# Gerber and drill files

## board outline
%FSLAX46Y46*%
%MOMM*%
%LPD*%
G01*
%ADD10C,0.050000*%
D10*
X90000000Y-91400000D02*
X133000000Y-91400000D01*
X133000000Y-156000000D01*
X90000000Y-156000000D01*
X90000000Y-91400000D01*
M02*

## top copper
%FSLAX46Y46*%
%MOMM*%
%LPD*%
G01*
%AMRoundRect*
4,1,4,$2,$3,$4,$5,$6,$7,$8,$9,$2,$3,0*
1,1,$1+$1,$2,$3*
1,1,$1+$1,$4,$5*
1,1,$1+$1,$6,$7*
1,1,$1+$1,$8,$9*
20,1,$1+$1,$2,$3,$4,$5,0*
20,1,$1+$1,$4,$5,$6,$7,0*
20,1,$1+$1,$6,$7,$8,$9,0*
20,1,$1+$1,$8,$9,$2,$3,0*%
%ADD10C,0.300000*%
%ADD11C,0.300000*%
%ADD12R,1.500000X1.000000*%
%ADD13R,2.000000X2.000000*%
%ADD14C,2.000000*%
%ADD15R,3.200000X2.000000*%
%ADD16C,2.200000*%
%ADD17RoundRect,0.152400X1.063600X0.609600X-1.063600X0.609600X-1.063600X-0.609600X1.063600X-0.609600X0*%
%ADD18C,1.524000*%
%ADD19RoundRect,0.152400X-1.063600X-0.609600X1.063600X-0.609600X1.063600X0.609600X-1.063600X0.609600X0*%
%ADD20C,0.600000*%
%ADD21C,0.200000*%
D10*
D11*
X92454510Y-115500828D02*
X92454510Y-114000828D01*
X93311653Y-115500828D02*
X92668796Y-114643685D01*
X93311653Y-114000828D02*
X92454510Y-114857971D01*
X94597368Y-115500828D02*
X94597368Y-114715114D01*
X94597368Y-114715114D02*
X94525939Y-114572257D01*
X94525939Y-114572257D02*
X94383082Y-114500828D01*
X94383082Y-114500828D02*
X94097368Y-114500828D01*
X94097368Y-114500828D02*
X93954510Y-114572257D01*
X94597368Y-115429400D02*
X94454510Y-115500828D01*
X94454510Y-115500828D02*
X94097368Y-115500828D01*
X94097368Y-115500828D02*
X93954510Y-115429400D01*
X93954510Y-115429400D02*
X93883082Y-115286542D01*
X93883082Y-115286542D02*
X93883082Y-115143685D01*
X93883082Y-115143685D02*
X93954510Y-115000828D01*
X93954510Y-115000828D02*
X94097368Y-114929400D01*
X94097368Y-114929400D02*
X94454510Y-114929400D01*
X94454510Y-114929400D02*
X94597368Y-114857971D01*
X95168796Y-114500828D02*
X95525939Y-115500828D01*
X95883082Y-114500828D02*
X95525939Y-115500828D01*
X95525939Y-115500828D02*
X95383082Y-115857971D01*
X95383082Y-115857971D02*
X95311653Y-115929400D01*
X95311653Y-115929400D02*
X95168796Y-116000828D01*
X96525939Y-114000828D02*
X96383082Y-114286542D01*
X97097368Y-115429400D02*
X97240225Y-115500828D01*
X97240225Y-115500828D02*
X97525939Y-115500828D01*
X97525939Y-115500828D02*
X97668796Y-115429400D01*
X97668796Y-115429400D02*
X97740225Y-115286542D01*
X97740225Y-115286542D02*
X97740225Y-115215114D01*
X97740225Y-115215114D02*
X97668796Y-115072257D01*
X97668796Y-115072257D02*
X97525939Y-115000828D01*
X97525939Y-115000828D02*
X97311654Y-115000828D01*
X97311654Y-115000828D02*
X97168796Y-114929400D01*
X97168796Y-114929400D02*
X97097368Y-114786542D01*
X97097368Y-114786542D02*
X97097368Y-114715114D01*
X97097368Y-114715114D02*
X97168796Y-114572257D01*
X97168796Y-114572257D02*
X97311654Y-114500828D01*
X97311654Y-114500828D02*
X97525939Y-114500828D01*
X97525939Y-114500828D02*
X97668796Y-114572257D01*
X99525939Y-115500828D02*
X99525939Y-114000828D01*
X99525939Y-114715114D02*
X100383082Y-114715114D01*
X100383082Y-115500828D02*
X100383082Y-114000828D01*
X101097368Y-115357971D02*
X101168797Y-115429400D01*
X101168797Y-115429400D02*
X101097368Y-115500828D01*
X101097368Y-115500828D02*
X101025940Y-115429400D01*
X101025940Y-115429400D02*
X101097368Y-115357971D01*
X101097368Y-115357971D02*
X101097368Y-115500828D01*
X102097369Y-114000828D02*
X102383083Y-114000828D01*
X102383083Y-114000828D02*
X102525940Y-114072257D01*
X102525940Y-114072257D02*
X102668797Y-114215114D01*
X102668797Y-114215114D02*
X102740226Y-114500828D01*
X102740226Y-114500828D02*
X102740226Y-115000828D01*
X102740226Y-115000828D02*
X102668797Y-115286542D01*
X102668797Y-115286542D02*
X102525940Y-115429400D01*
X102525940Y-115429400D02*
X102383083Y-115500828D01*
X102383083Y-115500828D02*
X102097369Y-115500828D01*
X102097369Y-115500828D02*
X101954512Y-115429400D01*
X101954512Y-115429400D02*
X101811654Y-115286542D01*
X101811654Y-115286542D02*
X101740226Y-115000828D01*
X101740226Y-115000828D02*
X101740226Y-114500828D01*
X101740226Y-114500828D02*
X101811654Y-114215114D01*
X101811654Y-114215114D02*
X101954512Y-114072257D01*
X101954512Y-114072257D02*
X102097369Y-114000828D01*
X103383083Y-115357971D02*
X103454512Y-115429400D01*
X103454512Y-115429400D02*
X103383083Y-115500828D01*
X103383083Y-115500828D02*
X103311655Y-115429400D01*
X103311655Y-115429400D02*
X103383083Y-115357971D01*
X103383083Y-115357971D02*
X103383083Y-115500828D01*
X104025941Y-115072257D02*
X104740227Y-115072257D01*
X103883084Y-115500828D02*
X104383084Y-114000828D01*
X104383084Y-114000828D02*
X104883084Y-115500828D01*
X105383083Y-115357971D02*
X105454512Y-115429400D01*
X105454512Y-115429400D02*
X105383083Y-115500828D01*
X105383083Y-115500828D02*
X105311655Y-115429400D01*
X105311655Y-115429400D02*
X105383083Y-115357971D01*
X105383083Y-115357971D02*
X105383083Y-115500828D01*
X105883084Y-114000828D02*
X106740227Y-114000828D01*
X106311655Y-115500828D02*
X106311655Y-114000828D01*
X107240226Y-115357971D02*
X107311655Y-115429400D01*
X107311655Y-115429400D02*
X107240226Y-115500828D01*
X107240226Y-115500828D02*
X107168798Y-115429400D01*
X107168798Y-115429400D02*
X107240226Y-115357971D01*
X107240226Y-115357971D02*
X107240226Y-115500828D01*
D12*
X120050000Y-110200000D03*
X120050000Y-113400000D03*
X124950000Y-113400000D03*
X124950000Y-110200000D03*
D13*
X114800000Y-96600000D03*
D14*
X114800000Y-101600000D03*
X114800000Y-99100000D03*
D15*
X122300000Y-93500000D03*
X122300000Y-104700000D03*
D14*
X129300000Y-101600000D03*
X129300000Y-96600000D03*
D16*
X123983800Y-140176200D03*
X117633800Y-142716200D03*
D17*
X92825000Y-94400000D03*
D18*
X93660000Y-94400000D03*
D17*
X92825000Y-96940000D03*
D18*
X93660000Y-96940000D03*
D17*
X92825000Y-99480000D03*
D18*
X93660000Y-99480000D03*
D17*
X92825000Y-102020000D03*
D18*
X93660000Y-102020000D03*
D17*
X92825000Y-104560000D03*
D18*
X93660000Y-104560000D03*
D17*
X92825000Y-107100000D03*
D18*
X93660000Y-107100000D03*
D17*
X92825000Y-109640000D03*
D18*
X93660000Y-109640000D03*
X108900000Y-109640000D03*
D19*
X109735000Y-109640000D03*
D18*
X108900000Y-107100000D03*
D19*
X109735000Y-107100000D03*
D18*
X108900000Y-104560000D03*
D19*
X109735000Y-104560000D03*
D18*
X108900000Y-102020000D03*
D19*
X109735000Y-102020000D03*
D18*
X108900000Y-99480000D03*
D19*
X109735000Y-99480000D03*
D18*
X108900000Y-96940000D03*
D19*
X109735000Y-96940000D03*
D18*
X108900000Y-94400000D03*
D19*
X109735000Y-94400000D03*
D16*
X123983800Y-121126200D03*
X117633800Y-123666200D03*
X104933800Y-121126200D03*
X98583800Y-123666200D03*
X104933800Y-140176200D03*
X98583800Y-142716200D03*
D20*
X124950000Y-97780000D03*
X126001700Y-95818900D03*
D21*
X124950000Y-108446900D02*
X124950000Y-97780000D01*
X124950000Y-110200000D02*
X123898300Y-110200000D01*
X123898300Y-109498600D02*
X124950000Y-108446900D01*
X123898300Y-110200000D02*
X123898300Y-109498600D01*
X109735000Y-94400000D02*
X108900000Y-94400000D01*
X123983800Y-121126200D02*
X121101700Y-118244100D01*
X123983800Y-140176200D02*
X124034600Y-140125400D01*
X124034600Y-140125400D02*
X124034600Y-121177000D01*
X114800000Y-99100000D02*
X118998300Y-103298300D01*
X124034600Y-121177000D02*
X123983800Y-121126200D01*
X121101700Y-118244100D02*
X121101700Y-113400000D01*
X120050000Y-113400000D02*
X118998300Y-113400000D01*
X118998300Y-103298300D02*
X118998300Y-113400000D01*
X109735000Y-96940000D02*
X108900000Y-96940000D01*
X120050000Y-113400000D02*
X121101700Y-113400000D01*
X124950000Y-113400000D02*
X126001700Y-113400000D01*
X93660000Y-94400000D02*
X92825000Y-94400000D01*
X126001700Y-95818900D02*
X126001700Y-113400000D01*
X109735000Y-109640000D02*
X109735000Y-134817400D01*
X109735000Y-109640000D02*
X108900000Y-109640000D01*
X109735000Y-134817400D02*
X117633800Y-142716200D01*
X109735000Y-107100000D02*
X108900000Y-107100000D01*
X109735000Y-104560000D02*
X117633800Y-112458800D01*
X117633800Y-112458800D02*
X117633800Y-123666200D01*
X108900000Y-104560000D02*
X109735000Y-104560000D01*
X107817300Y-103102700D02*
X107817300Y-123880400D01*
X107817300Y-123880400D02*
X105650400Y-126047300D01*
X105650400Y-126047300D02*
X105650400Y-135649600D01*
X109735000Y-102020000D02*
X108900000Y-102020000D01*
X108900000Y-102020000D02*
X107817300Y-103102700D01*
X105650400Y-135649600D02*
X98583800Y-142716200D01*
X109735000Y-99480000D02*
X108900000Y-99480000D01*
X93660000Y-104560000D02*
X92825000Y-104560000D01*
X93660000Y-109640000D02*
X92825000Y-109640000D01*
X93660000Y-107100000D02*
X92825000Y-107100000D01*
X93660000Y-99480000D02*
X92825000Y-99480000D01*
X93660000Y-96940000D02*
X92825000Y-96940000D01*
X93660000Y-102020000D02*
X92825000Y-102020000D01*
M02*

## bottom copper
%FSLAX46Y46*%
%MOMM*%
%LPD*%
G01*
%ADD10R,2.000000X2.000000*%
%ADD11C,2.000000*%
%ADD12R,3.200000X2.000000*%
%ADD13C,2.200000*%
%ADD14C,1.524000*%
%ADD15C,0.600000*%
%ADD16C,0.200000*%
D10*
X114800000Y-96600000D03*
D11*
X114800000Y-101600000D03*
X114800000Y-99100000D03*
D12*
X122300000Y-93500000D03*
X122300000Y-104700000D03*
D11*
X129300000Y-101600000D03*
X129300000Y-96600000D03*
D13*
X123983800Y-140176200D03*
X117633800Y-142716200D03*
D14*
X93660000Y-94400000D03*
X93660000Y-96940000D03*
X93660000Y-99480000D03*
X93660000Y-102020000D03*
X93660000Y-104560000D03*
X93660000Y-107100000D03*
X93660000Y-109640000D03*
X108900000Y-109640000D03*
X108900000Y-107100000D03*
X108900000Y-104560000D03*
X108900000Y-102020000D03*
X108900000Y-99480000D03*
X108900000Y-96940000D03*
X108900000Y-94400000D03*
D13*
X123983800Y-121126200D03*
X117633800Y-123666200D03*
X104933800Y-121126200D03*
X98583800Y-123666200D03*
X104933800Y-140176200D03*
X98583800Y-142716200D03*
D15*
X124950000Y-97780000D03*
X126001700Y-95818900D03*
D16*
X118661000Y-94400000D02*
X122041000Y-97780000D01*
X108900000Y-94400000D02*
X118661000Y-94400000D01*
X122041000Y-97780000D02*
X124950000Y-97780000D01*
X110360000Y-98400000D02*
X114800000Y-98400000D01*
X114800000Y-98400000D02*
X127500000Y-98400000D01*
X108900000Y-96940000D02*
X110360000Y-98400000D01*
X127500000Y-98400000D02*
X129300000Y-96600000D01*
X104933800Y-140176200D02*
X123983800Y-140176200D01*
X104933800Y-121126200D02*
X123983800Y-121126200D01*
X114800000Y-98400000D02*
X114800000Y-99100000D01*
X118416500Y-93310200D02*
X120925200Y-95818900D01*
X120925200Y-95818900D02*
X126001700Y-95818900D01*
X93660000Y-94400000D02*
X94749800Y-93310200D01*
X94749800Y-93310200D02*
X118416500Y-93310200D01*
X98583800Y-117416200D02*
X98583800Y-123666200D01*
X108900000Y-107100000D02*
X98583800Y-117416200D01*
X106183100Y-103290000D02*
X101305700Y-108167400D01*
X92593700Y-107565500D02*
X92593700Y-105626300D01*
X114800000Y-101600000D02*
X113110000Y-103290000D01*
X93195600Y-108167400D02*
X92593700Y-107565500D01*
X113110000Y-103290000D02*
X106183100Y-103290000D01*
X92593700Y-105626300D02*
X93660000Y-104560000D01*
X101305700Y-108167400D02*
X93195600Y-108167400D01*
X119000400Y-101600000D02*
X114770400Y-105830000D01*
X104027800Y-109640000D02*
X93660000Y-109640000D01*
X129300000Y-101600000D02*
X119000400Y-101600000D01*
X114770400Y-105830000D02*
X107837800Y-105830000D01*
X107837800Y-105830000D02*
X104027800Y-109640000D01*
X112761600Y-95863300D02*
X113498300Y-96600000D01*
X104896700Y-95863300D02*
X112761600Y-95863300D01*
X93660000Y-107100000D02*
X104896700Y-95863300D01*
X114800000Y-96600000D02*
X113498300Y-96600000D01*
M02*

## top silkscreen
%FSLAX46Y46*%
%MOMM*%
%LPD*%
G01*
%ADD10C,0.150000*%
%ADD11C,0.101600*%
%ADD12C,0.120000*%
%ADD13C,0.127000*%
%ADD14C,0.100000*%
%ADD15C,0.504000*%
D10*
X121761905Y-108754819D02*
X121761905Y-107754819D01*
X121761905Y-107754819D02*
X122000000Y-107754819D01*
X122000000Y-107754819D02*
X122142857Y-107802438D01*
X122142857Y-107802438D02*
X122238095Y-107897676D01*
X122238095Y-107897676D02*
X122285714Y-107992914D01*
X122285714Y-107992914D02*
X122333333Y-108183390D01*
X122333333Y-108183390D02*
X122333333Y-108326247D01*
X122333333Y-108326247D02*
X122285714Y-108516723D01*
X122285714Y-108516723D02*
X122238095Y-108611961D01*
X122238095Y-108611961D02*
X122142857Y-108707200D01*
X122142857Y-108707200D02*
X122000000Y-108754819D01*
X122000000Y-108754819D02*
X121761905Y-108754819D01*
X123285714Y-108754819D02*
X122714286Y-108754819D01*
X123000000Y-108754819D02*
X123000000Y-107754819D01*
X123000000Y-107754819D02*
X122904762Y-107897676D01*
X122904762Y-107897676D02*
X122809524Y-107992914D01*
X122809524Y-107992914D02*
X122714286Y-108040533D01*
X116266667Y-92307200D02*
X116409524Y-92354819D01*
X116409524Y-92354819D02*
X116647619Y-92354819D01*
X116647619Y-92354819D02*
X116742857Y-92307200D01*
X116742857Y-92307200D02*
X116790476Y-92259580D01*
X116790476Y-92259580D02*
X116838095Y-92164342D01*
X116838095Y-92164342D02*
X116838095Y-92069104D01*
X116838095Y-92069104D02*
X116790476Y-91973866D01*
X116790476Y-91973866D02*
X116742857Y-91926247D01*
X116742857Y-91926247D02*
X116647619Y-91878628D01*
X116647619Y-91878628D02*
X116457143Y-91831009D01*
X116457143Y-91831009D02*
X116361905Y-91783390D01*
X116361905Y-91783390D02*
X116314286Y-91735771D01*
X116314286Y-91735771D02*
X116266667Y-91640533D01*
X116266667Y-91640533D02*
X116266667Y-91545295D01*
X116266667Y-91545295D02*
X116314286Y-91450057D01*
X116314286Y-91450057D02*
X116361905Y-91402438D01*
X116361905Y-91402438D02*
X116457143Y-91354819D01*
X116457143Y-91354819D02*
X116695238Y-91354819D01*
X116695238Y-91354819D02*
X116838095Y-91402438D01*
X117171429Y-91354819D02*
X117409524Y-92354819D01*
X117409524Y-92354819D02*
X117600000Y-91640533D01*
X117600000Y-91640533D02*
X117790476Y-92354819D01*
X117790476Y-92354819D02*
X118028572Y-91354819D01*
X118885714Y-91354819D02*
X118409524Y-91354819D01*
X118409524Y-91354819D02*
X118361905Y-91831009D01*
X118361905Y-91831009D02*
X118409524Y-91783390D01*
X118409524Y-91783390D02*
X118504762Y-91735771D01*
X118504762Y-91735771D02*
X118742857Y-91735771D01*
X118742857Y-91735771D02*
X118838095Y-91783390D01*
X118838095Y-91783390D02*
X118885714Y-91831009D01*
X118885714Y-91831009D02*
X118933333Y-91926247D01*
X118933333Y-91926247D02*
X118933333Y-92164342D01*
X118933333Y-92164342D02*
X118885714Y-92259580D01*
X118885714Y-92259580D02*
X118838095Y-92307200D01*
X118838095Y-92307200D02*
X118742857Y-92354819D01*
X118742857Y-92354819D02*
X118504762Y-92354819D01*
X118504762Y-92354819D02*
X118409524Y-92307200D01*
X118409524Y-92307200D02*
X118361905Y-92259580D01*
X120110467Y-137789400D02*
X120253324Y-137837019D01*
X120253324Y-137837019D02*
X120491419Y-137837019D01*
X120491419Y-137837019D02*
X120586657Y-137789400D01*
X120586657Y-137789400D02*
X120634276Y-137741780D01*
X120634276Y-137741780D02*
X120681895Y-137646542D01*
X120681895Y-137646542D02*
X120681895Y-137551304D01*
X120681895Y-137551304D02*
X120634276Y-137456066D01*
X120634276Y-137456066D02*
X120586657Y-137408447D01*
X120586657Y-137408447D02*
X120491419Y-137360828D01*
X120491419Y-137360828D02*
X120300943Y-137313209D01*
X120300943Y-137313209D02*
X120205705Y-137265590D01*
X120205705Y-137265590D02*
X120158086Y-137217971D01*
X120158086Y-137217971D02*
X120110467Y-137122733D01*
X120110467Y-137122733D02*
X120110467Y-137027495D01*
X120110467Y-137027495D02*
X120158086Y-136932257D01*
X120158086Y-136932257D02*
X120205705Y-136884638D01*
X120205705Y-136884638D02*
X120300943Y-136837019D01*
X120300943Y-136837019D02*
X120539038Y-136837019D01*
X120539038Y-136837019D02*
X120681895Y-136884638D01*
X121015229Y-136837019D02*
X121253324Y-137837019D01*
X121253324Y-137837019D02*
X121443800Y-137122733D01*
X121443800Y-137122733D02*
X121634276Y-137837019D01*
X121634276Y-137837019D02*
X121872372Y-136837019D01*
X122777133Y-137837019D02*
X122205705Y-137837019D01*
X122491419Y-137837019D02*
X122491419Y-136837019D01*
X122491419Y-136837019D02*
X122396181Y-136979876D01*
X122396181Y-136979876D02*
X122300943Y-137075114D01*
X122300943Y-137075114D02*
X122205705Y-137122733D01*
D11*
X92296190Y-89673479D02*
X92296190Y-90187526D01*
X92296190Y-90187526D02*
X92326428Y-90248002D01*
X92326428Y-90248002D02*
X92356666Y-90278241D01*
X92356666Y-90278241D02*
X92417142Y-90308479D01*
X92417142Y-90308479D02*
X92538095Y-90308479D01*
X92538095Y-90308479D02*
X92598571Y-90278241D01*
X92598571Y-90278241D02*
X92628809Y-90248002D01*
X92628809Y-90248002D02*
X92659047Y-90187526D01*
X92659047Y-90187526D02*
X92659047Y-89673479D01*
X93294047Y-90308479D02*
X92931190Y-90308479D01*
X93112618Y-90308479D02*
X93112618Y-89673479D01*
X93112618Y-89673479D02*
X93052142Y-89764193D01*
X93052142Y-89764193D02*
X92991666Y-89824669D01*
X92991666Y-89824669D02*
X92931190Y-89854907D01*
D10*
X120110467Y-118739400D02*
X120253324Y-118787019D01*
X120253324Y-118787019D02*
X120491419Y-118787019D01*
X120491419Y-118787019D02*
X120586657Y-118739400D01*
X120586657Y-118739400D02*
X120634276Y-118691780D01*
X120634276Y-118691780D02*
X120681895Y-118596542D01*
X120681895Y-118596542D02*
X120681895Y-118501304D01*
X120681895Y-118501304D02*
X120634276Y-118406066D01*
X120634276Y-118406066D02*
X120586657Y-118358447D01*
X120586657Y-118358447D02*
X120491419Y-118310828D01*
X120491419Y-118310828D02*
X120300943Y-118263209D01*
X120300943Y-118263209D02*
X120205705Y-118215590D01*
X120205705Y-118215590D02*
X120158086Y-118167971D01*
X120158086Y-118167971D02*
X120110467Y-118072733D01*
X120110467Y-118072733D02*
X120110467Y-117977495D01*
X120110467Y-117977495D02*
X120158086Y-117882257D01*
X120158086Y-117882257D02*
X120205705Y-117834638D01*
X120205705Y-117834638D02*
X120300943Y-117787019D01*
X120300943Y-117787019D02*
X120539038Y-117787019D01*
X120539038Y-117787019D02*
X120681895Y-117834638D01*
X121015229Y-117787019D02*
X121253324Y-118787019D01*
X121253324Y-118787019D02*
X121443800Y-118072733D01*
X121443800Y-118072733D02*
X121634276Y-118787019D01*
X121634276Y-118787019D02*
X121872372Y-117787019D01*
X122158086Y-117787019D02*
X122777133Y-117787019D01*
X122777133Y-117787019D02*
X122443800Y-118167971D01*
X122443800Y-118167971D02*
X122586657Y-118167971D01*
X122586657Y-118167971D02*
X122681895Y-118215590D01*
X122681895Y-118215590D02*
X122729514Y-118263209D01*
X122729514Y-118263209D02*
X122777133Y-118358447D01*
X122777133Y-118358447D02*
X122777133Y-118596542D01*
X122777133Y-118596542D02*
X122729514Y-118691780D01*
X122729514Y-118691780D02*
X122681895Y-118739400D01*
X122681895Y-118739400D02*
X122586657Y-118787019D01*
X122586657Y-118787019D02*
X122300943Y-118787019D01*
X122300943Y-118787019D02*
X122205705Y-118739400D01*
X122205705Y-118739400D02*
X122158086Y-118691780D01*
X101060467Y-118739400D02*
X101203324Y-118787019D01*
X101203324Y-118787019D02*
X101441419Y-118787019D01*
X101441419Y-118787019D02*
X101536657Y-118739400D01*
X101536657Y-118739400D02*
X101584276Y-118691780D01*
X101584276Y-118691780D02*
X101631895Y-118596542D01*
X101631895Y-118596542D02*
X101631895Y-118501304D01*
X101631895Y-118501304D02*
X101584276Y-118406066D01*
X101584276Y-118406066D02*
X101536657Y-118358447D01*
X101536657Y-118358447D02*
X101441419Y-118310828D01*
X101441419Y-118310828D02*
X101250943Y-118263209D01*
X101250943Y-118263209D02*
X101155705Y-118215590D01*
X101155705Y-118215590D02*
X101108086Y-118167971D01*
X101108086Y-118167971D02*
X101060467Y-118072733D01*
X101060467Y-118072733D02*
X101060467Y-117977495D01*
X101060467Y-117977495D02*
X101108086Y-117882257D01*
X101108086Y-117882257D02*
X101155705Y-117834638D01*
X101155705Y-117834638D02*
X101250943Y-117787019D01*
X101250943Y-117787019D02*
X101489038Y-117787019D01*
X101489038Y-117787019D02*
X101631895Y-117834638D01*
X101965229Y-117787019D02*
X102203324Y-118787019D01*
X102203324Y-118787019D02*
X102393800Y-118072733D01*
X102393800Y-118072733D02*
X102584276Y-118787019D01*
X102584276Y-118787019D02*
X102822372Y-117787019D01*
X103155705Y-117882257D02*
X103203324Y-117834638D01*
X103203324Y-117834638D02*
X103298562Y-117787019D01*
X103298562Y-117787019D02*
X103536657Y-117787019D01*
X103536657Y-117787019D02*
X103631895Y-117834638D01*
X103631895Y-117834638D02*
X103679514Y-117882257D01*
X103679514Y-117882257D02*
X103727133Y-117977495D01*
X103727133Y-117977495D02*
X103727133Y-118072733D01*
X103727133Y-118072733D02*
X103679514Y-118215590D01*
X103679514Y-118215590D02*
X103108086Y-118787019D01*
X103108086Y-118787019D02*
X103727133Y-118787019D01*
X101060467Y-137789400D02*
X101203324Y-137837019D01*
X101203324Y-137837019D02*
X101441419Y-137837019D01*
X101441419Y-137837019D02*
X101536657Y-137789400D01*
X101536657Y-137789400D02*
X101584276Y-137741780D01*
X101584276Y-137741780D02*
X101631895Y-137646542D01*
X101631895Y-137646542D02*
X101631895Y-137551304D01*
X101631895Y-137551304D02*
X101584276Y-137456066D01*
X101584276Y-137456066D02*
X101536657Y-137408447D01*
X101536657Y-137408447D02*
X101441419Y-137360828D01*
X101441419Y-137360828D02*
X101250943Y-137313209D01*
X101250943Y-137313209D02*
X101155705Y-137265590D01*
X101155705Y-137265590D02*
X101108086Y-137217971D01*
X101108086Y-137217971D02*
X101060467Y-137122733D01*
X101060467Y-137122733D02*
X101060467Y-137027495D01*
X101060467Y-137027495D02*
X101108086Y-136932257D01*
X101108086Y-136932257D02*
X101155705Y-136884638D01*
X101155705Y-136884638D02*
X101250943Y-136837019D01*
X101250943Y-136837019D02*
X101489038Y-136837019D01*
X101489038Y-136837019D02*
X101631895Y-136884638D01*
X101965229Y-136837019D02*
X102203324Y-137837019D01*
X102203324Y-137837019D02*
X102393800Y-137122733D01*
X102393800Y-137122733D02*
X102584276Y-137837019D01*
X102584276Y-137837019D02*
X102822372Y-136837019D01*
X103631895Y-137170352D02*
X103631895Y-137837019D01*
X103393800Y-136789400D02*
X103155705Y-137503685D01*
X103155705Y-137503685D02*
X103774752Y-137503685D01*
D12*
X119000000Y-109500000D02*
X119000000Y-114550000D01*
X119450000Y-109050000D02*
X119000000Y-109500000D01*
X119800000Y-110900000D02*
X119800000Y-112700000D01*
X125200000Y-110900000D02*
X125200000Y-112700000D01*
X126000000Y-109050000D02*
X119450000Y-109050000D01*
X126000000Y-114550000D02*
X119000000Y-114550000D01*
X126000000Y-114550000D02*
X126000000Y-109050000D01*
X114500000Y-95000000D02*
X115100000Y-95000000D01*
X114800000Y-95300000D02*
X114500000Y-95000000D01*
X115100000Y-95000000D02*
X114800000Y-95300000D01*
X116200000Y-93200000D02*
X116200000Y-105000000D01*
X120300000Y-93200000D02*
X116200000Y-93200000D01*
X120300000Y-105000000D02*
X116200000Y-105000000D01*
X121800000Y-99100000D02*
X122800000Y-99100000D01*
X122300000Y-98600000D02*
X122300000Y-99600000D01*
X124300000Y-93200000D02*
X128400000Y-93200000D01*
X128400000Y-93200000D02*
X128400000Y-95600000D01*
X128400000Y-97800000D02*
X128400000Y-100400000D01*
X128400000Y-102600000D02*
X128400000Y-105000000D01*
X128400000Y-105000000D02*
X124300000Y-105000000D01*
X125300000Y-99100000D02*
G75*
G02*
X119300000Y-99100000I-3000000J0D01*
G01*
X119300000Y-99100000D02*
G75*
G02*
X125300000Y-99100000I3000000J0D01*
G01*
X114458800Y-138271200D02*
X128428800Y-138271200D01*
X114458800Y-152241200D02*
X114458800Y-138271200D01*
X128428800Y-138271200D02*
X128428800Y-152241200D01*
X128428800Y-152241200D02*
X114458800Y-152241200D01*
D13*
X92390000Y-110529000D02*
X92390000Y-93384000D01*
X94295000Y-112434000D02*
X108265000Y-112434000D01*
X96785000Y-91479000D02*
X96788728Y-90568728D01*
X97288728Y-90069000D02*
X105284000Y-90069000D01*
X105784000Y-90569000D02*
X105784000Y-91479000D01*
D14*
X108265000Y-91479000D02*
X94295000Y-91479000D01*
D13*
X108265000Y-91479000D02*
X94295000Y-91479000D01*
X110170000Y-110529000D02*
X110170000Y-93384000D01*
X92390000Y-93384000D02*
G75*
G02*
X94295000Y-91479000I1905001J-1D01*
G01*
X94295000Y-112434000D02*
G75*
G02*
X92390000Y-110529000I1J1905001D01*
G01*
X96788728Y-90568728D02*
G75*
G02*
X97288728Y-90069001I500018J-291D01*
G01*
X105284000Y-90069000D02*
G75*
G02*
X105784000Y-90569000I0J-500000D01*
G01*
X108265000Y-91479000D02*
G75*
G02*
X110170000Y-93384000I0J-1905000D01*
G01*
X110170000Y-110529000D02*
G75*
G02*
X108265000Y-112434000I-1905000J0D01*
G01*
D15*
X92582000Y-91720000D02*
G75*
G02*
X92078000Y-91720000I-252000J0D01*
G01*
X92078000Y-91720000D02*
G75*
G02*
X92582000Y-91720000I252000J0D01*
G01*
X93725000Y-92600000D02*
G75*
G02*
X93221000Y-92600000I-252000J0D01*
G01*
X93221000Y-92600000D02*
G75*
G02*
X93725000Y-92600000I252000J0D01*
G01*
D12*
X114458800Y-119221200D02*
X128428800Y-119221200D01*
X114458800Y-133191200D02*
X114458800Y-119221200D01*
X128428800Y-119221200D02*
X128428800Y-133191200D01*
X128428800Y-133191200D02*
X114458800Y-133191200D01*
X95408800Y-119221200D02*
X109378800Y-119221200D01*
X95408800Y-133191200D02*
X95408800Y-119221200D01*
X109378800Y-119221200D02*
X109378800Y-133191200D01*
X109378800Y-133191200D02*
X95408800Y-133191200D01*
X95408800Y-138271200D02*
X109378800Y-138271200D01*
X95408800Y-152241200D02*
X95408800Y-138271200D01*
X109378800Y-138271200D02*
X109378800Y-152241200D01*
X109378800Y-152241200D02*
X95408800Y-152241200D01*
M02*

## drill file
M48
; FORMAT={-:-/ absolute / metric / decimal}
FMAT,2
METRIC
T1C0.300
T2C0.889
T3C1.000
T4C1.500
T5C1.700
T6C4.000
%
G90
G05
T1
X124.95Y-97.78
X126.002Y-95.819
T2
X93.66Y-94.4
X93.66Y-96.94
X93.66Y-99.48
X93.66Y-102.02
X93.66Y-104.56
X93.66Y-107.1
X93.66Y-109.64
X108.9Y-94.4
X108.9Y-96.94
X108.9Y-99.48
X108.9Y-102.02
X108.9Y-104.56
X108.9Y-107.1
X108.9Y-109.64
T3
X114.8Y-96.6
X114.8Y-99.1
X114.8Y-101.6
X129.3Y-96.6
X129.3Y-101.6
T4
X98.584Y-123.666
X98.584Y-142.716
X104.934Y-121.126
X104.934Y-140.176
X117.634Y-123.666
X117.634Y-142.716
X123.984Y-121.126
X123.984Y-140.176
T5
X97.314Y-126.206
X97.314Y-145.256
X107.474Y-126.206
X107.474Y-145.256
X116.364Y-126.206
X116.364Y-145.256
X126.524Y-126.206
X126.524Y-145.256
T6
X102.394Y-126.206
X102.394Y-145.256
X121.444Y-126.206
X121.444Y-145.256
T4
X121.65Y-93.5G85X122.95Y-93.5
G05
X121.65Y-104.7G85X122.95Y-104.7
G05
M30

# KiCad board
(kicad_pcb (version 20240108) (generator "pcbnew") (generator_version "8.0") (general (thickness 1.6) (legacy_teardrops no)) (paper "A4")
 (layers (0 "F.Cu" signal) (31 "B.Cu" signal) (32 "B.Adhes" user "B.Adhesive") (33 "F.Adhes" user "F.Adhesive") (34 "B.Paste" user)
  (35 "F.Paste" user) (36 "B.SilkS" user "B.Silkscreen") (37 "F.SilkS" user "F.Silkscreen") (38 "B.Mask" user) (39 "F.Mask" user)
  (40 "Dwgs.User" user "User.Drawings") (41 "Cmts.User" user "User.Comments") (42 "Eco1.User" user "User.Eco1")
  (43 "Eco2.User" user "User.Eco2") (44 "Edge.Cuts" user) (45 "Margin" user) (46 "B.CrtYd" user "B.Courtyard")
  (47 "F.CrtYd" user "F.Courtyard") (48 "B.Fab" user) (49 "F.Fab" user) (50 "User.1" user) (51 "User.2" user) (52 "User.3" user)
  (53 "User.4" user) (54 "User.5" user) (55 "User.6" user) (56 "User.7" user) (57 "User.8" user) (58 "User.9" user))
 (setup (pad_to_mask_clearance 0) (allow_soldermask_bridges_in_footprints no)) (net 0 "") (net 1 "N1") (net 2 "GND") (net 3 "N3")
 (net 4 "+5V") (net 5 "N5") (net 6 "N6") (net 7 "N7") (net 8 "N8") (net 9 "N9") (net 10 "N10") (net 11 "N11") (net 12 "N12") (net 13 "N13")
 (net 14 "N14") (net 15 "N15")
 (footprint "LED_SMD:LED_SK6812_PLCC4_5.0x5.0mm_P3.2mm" (layer "F.Cu") (at 122.5 111.8)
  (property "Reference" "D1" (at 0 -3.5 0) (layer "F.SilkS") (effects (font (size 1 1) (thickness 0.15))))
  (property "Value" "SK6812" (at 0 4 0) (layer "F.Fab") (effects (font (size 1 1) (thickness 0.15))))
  (fp_line (start -3.5 -2.3) (end -3.5 2.75) (stroke (width 0.12) (type default)) (layer "F.SilkS"))
  (fp_line (start -3.05 -2.75) (end -3.5 -2.3) (stroke (width 0.12) (type default)) (layer "F.SilkS"))
  (fp_line (start -2.7 -0.9) (end -2.7 0.9) (stroke (width 0.12) (type default)) (layer "F.SilkS"))
  (fp_line (start 2.7 -0.9) (end 2.7 0.9) (stroke (width 0.12) (type default)) (layer "F.SilkS"))
  (fp_line (start 3.5 -2.75) (end -3.05 -2.75) (stroke (width 0.12) (type solid)) (layer "F.SilkS"))
  (fp_line (start 3.5 2.75) (end -3.5 2.75) (stroke (width 0.12) (type solid)) (layer "F.SilkS"))
  (fp_line (start 3.5 2.75) (end 3.5 -2.75) (stroke (width 0.12) (type default)) (layer "F.SilkS"))
  (pad "1" smd rect (at -2.45 -1.6 180) (size 1.5 1) (layers "F.Cu" "F.Paste" "F.Mask") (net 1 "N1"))
  (pad "2" smd rect (at -2.45 1.6 180) (size 1.5 1) (layers "F.Cu" "F.Paste" "F.Mask") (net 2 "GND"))
  (pad "3" smd rect (at 2.45 1.6 180) (size 1.5 1) (layers "F.Cu" "F.Paste" "F.Mask") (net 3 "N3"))
  (pad "4" smd rect (at 2.45 -1.6 180) (size 1.5 1) (layers "F.Cu" "F.Paste" "F.Mask") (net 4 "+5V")))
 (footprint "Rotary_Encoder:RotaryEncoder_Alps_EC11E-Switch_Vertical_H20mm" (layer "F.Cu") (at 114.8 96.6)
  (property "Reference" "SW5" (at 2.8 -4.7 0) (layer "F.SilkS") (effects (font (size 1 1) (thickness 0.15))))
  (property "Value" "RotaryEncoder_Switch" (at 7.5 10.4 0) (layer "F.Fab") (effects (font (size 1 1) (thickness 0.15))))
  (fp_line (start -0.3 -1.6) (end 0.3 -1.6) (stroke (width 0.12) (type solid)) (layer "F.SilkS"))
  (fp_line (start 0 -1.3) (end -0.3 -1.6) (stroke (width 0.12) (type solid)) (layer "F.SilkS"))
  (fp_line (start 0.3 -1.6) (end 0 -1.3) (stroke (width 0.12) (type solid)) (layer "F.SilkS"))
  (fp_line (start 1.4 -3.4) (end 1.4 8.4) (stroke (width 0.12) (type solid)) (layer "F.SilkS"))
  (fp_line (start 5.5 -3.4) (end 1.4 -3.4) (stroke (width 0.12) (type solid)) (layer "F.SilkS"))
  (fp_line (start 5.5 8.4) (end 1.4 8.4) (stroke (width 0.12) (type solid)) (layer "F.SilkS"))
  (fp_line (start 7 2.5) (end 8 2.5) (stroke (width 0.12) (type solid)) (layer "F.SilkS"))
  (fp_line (start 7.5 2) (end 7.5 3) (stroke (width 0.12) (type solid)) (layer "F.SilkS"))
  (fp_line (start 9.5 -3.4) (end 13.6 -3.4) (stroke (width 0.12) (type solid)) (layer "F.SilkS"))
  (fp_line (start 13.6 -3.4) (end 13.6 -1) (stroke (width 0.12) (type solid)) (layer "F.SilkS"))
  (fp_line (start 13.6 1.2) (end 13.6 3.8) (stroke (width 0.12) (type solid)) (layer "F.SilkS"))
  (fp_line (start 13.6 6) (end 13.6 8.4) (stroke (width 0.12) (type solid)) (layer "F.SilkS"))
  (fp_line (start 13.6 8.4) (end 9.5 8.4) (stroke (width 0.12) (type solid)) (layer "F.SilkS"))
  (fp_circle (center 7.5 2.5) (end 10.5 2.5) (stroke (width 0.12) (type solid)) (fill none) (layer "F.SilkS"))
  (pad "A" thru_hole rect (at 0 0) (size 2 2) (drill 1) (layers "*.Cu" "*.Mask") (remove_unused_layers no) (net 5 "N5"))
  (pad "B" thru_hole circle (at 0 5) (size 2 2) (drill 1) (layers "*.Cu" "*.Mask") (remove_unused_layers no) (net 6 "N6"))
  (pad "C" thru_hole circle (at 0 2.5) (size 2 2) (drill 1) (layers "*.Cu" "*.Mask") (remove_unused_layers no) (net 2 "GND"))
  (pad "MP" thru_hole rect (at 7.5 -3.1) (size 3.2 2) (drill oval 2.8 1.5) (layers "*.Cu" "*.Mask") (remove_unused_layers no))
  (pad "MP" thru_hole rect (at 7.5 8.1) (size 3.2 2) (drill oval 2.8 1.5) (layers "*.Cu" "*.Mask") (remove_unused_layers no))
  (pad "S1" thru_hole circle (at 14.5 5) (size 2 2) (drill 1) (layers "*.Cu" "*.Mask") (remove_unused_layers no) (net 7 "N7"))
  (pad "S2" thru_hole circle (at 14.5 0) (size 2 2) (drill 1) (layers "*.Cu" "*.Mask") (remove_unused_layers no) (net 2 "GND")))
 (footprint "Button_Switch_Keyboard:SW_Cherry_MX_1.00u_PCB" (layer "F.Cu") (at 123.9838 140.1762)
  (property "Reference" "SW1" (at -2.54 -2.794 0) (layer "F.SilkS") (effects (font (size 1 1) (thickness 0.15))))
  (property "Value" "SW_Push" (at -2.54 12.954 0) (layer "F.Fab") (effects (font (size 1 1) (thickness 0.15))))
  (fp_line (start -9.525 -1.905) (end 4.445 -1.905) (stroke (width 0.12) (type solid)) (layer "F.SilkS"))
  (fp_line (start -9.525 12.065) (end -9.525 -1.905) (stroke (width 0.12) (type solid)) (layer "F.SilkS"))
  (fp_line (start 4.445 -1.905) (end 4.445 12.065) (stroke (width 0.12) (type solid)) (layer "F.SilkS"))
  (fp_line (start 4.445 12.065) (end -9.525 12.065) (stroke (width 0.12) (type solid)) (layer "F.SilkS"))
  (pad "" np_thru_hole circle (at -7.62 5.08) (size 1.7 1.7) (drill 1.7) (layers "*.Cu" "*.Mask"))
  (pad "" np_thru_hole circle (at -2.54 5.08) (size 4 4) (drill 4) (layers "*.Cu" "*.Mask"))
  (pad "" np_thru_hole circle (at 2.54 5.08) (size 1.7 1.7) (drill 1.7) (layers "*.Cu" "*.Mask"))
  (pad "1" thru_hole circle (at 0 0) (size 2.2 2.2) (drill 1.5) (layers "*.Cu" "*.Mask") (remove_unused_layers no) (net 2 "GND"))
  (pad "2" thru_hole circle (at -6.35 2.54) (size 2.2 2.2) (drill 1.5) (layers "*.Cu" "*.Mask") (remove_unused_layers no) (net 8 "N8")))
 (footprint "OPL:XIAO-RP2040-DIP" (layer "F.Cu") (at 101.28 102.02)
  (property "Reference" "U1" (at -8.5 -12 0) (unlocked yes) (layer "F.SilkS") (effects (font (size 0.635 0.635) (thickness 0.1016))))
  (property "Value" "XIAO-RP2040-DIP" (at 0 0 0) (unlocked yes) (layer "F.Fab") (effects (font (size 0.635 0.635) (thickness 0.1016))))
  (fp_line (start -8.89 8.509) (end -8.89 -8.636) (stroke (width 0.127) (type solid)) (layer "F.SilkS"))
  (fp_line (start -6.985 10.414) (end 6.985 10.414) (stroke (width 0.127) (type solid)) (layer "F.SilkS"))
  (fp_line (start -4.495 -10.541) (end -4.491272 -11.451272) (stroke (width 0.127) (type solid)) (layer "F.SilkS"))
  (fp_line (start -3.991272 -11.951) (end 4.004 -11.951) (stroke (width 0.127) (type solid)) (layer "F.SilkS"))
  (fp_line (start 4.504 -11.451) (end 4.504 -10.541) (stroke (width 0.127) (type solid)) (layer "F.SilkS"))
  (fp_line (start 6.985 -10.541) (end -6.985 -10.541) (stroke (width 0.1) (type solid)) (layer "F.SilkS"))
  (fp_line (start 6.985 -10.541) (end -6.985 -10.541) (stroke (width 0.127) (type solid)) (layer "F.SilkS"))
  (fp_line (start 8.89 8.509) (end 8.89 -8.636) (stroke (width 0.127) (type solid)) (layer "F.SilkS"))
  (fp_arc (start -8.89 -8.636) (mid -8.332038 -9.983038) (end -6.985 -10.541) (stroke (width 0.127) (type solid)) (layer "F.SilkS"))
  (fp_arc (start -6.985 10.414) (mid -8.332038 9.856038) (end -8.89 8.509) (stroke (width 0.127) (type solid)) (layer "F.SilkS"))
  (fp_arc (start -4.491272 -11.451272) (mid -4.344724 -11.804644) (end -3.991272 -11.951) (stroke (width 0.127) (type default))
   (layer "F.SilkS"))
  (fp_arc (start 4.004 -11.951) (mid 4.357553 -11.804553) (end 4.504 -11.451) (stroke (width 0.127) (type default)) (layer "F.SilkS"))
  (fp_arc (start 6.985 -10.541) (mid 8.332038 -9.983038) (end 8.89 -8.636) (stroke (width 0.127) (type solid)) (layer "F.SilkS"))
  (fp_arc (start 8.89 8.509) (mid 8.332038 9.856038) (end 6.985 10.414) (stroke (width 0.127) (type solid)) (layer "F.SilkS"))
  (fp_circle (center -8.95 -10.3) (end -8.95 -10.554) (stroke (width 0.5) (type solid)) (fill solid) (layer "F.SilkS"))
  (fp_circle (center -7.807 -9.42) (end -7.807 -9.674) (stroke (width 0.5) (type solid)) (fill solid) (layer "F.SilkS"))
  (pad "1" smd roundrect (at -8.455 -7.62 180) (size 2.432 1.524) (layers "F.Cu" "F.Mask") (roundrect_rratio 0.1) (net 3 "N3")
   (thermal_bridge_angle 45))
  (pad "1" thru_hole circle (at -7.62 -7.62 180) (size 1.524 1.524) (drill 0.889) (layers "*.Cu" "*.Mask") (remove_unused_layers no)
   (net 3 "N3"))
  (pad "2" smd roundrect (at -8.455 -5.08 180) (size 2.432 1.524) (layers "F.Cu" "F.Mask") (roundrect_rratio 0.1) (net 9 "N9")
   (thermal_bridge_angle 45))
  (pad "2" thru_hole circle (at -7.62 -5.08 180) (size 1.524 1.524) (drill 0.889) (layers "*.Cu" "*.Mask") (remove_unused_layers no)
   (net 9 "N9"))
  (pad "3" smd roundrect (at -8.455 -2.54 180) (size 2.432 1.524) (layers "F.Cu" "F.Mask") (roundrect_rratio 0.1) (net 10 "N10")
   (thermal_bridge_angle 45))
  (pad "3" thru_hole circle (at -7.62 -2.54 180) (size 1.524 1.524) (drill 0.889) (layers "*.Cu" "*.Mask") (remove_unused_layers no)
   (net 10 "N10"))
  (pad "4" smd roundrect (at -8.455 0 180) (size 2.432 1.524) (layers "F.Cu" "F.Mask") (roundrect_rratio 0.1) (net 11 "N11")
   (thermal_bridge_angle 45))
  (pad "4" thru_hole circle (at -7.62 0 180) (size 1.524 1.524) (drill 0.889) (layers "*.Cu" "*.Mask") (remove_unused_layers no)
   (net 11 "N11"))
  (pad "5" smd roundrect (at -8.455 2.54 180) (size 2.432 1.524) (layers "F.Cu" "F.Mask") (roundrect_rratio 0.1) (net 6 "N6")
   (thermal_bridge_angle 45))
  (pad "5" thru_hole circle (at -7.62 2.54 180) (size 1.524 1.524) (drill 0.889) (layers "*.Cu" "*.Mask") (remove_unused_layers no)
   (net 6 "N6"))
  (pad "6" smd roundrect (at -8.455 5.08 180) (size 2.432 1.524) (layers "F.Cu" "F.Mask") (roundrect_rratio 0.1) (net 5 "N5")
   (thermal_bridge_angle 45))
  (pad "6" thru_hole circle (at -7.62 5.08 180) (size 1.524 1.524) (drill 0.889) (layers "*.Cu" "*.Mask") (remove_unused_layers no)
   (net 5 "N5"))
  (pad "7" smd roundrect (at -8.455 7.62 180) (size 2.432 1.524) (layers "F.Cu" "F.Mask") (roundrect_rratio 0.1) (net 7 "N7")
   (thermal_bridge_angle 45))
  (pad "7" thru_hole circle (at -7.62 7.62 180) (size 1.524 1.524) (drill 0.889) (layers "*.Cu" "*.Mask") (remove_unused_layers no)
   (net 7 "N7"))
  (pad "8" thru_hole circle (at 7.62 7.62) (size 1.524 1.524) (drill 0.889) (layers "*.Cu" "*.Mask") (remove_unused_layers no) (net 8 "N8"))
  (pad "8" smd roundrect (at 8.455 7.62) (size 2.432 1.524) (layers "F.Cu" "F.Mask") (roundrect_rratio 0.1) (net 8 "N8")
   (thermal_bridge_angle 45))
  (pad "9" thru_hole circle (at 7.62 5.08) (size 1.524 1.524) (drill 0.889) (layers "*.Cu" "*.Mask") (remove_unused_layers no)
   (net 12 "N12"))
  (pad "9" smd roundrect (at 8.455 5.08) (size 2.432 1.524) (layers "F.Cu" "F.Mask") (roundrect_rratio 0.1) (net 12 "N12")
   (thermal_bridge_angle 45))
  (pad "10" thru_hole circle (at 7.62 2.54) (size 1.524 1.524) (drill 0.889) (layers "*.Cu" "*.Mask") (remove_unused_layers no)
   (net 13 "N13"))
  (pad "10" smd roundrect (at 8.455 2.54) (size 2.432 1.524) (layers "F.Cu" "F.Mask") (roundrect_rratio 0.1) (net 13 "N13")
   (thermal_bridge_angle 45))
  (pad "11" thru_hole circle (at 7.62 0) (size 1.524 1.524) (drill 0.889) (layers "*.Cu" "*.Mask") (remove_unused_layers no) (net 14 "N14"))
  (pad "11" smd roundrect (at 8.455 0) (size 2.432 1.524) (layers "F.Cu" "F.Mask") (roundrect_rratio 0.1) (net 14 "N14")
   (thermal_bridge_angle 45))
  (pad "12" thru_hole circle (at 7.62 -2.54) (size 1.524 1.524) (drill 0.889) (layers "*.Cu" "*.Mask") (remove_unused_layers no)
   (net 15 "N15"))
  (pad "12" smd roundrect (at 8.455 -2.54) (size 2.432 1.524) (layers "F.Cu" "F.Mask") (roundrect_rratio 0.1) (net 15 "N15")
   (thermal_bridge_angle 45))
  (pad "13" thru_hole circle (at 7.62 -5.08) (size 1.524 1.524) (drill 0.889) (layers "*.Cu" "*.Mask") (remove_unused_layers no)
   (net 2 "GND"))
  (pad "13" smd roundrect (at 8.455 -5.08) (size 2.432 1.524) (layers "F.Cu" "F.Mask") (roundrect_rratio 0.1) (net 2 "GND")
   (thermal_bridge_angle 45))
  (pad "14" thru_hole circle (at 7.62 -7.62) (size 1.524 1.524) (drill 0.889) (layers "*.Cu" "*.Mask") (remove_unused_layers no)
   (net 4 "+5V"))
  (pad "14" smd roundrect (at 8.455 -7.62) (size 2.432 1.524) (layers "F.Cu" "F.Mask") (roundrect_rratio 0.1) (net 4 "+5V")
   (thermal_bridge_angle 45)))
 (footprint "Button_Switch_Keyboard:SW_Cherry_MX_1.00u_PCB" (layer "F.Cu") (at 123.9838 121.1262)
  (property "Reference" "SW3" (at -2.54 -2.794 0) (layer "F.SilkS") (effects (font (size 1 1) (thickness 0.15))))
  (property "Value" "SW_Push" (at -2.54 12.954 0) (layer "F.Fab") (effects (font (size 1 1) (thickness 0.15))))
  (fp_line (start -9.525 -1.905) (end 4.445 -1.905) (stroke (width 0.12) (type solid)) (layer "F.SilkS"))
  (fp_line (start -9.525 12.065) (end -9.525 -1.905) (stroke (width 0.12) (type solid)) (layer "F.SilkS"))
  (fp_line (start 4.445 -1.905) (end 4.445 12.065) (stroke (width 0.12) (type solid)) (layer "F.SilkS"))
  (fp_line (start 4.445 12.065) (end -9.525 12.065) (stroke (width 0.12) (type solid)) (layer "F.SilkS"))
  (pad "" np_thru_hole circle (at -7.62 5.08) (size 1.7 1.7) (drill 1.7) (layers "*.Cu" "*.Mask"))
  (pad "" np_thru_hole circle (at -2.54 5.08) (size 4 4) (drill 4) (layers "*.Cu" "*.Mask"))
  (pad "" np_thru_hole circle (at 2.54 5.08) (size 1.7 1.7) (drill 1.7) (layers "*.Cu" "*.Mask"))
  (pad "1" thru_hole circle (at 0 0) (size 2.2 2.2) (drill 1.5) (layers "*.Cu" "*.Mask") (remove_unused_layers no) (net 2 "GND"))
  (pad "2" thru_hole circle (at -6.35 2.54) (size 2.2 2.2) (drill 1.5) (layers "*.Cu" "*.Mask") (remove_unused_layers no) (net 13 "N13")))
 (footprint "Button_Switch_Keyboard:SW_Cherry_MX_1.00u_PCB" (layer "F.Cu") (at 104.9338 121.1262)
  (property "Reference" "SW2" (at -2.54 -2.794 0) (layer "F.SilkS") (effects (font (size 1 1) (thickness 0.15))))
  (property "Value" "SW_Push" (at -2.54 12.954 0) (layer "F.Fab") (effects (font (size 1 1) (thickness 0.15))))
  (fp_line (start -9.525 -1.905) (end 4.445 -1.905) (stroke (width 0.12) (type solid)) (layer "F.SilkS"))
  (fp_line (start -9.525 12.065) (end -9.525 -1.905) (stroke (width 0.12) (type solid)) (layer "F.SilkS"))
  (fp_line (start 4.445 -1.905) (end 4.445 12.065) (stroke (width 0.12) (type solid)) (layer "F.SilkS"))
  (fp_line (start 4.445 12.065) (end -9.525 12.065) (stroke (width 0.12) (type solid)) (layer "F.SilkS"))
  (pad "" np_thru_hole circle (at -7.62 5.08) (size 1.7 1.7) (drill 1.7) (layers "*.Cu" "*.Mask"))
  (pad "" np_thru_hole circle (at -2.54 5.08) (size 4 4) (drill 4) (layers "*.Cu" "*.Mask"))
  (pad "" np_thru_hole circle (at 2.54 5.08) (size 1.7 1.7) (drill 1.7) (layers "*.Cu" "*.Mask"))
  (pad "1" thru_hole circle (at 0 0) (size 2.2 2.2) (drill 1.5) (layers "*.Cu" "*.Mask") (remove_unused_layers no) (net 2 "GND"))
  (pad "2" thru_hole circle (at -6.35 2.54) (size 2.2 2.2) (drill 1.5) (layers "*.Cu" "*.Mask") (remove_unused_layers no) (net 12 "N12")))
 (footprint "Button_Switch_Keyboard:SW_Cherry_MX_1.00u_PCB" (layer "F.Cu") (at 104.9338 140.1762)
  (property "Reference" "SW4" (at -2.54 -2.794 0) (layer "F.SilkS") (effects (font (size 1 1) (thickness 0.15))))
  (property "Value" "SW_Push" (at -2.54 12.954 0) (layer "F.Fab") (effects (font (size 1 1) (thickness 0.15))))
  (fp_line (start -9.525 -1.905) (end 4.445 -1.905) (stroke (width 0.12) (type solid)) (layer "F.SilkS"))
  (fp_line (start -9.525 12.065) (end -9.525 -1.905) (stroke (width 0.12) (type solid)) (layer "F.SilkS"))
  (fp_line (start 4.445 -1.905) (end 4.445 12.065) (stroke (width 0.12) (type solid)) (layer "F.SilkS"))
  (fp_line (start 4.445 12.065) (end -9.525 12.065) (stroke (width 0.12) (type solid)) (layer "F.SilkS"))
  (pad "" np_thru_hole circle (at -7.62 5.08) (size 1.7 1.7) (drill 1.7) (layers "*.Cu" "*.Mask"))
  (pad "" np_thru_hole circle (at -2.54 5.08) (size 4 4) (drill 4) (layers "*.Cu" "*.Mask"))
  (pad "" np_thru_hole circle (at 2.54 5.08) (size 1.7 1.7) (drill 1.7) (layers "*.Cu" "*.Mask"))
  (pad "1" thru_hole circle (at 0 0) (size 2.2 2.2) (drill 1.5) (layers "*.Cu" "*.Mask") (remove_unused_layers no) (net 2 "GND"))
  (pad "2" thru_hole circle (at -6.35 2.54) (size 2.2 2.2) (drill 1.5) (layers "*.Cu" "*.Mask") (remove_unused_layers no) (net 14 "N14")))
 (gr_rect (start 90 91.4) (end 133 156) (stroke (width 0.05) (type default)) (fill none) (layer "Edge.Cuts"))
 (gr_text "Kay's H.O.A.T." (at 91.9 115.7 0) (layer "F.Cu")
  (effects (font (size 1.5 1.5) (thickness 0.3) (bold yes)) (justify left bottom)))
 (segment (start 124.95 108.4469) (end 124.95 97.78) (width 0.2) (layer "F.Cu") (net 4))
 (segment (start 124.95 110.2) (end 123.8983 110.2) (width 0.2) (layer "F.Cu") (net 4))
 (segment (start 123.8983 109.4986) (end 124.95 108.4469) (width 0.2) (layer "F.Cu") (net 4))
 (segment (start 123.8983 110.2) (end 123.8983 109.4986) (width 0.2) (layer "F.Cu") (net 4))
 (segment (start 109.735 94.4) (end 108.9 94.4) (width 0.2) (layer "F.Cu") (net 4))
 (via (at 124.95 97.78) (size 0.6) (drill 0.3) (layers "F.Cu" "B.Cu") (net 4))
 (segment (start 118.661 94.4) (end 122.041 97.78) (width 0.2) (layer "B.Cu") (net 4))
 (segment (start 108.9 94.4) (end 118.661 94.4) (width 0.2) (layer "B.Cu") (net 4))
 (segment (start 122.041 97.78) (end 124.95 97.78) (width 0.2) (layer "B.Cu") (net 4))
 (segment (start 123.9838 121.1262) (end 121.1017 118.2441) (width 0.2) (layer "F.Cu") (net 2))
 (segment (start 123.9838 140.1762) (end 124.0346 140.1254) (width 0.2) (layer "F.Cu") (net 2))
 (segment (start 124.0346 140.1254) (end 124.0346 121.177) (width 0.2) (layer "F.Cu") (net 2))
 (segment (start 114.8 99.1) (end 118.9983 103.2983) (width 0.2) (layer "F.Cu") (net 2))
 (segment (start 124.0346 121.177) (end 123.9838 121.1262) (width 0.2) (layer "F.Cu") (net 2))
 (segment (start 121.1017 118.2441) (end 121.1017 113.4) (width 0.2) (layer "F.Cu") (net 2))
 (segment (start 120.05 113.4) (end 118.9983 113.4) (width 0.2) (layer "F.Cu") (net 2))
 (segment (start 118.9983 103.2983) (end 118.9983 113.4) (width 0.2) (layer "F.Cu") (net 2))
 (segment (start 109.735 96.94) (end 108.9 96.94) (width 0.2) (layer "F.Cu") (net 2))
 (segment (start 120.05 113.4) (end 121.1017 113.4) (width 0.2) (layer "F.Cu") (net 2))
 (segment (start 110.36 98.4) (end 114.8 98.4) (width 0.2) (layer "B.Cu") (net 2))
 (segment (start 114.8 98.4) (end 127.5 98.4) (width 0.2) (layer "B.Cu") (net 2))
 (segment (start 108.9 96.94) (end 110.36 98.4) (width 0.2) (layer "B.Cu") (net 2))
 (segment (start 127.5 98.4) (end 129.3 96.6) (width 0.2) (layer "B.Cu") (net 2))
 (segment (start 104.9338 140.1762) (end 123.9838 140.1762) (width 0.2) (layer "B.Cu") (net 2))
 (segment (start 104.9338 121.1262) (end 123.9838 121.1262) (width 0.2) (layer "B.Cu") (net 2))
 (segment (start 114.8 98.4) (end 114.8 99.1) (width 0.2) (layer "B.Cu") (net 2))
 (segment (start 124.95 113.4) (end 126.0017 113.4) (width 0.2) (layer "F.Cu") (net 3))
 (segment (start 93.66 94.4) (end 92.825 94.4) (width 0.2) (layer "F.Cu") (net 3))
 (segment (start 126.0017 95.8189) (end 126.0017 113.4) (width 0.2) (layer "F.Cu") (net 3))
 (via (at 126.0017 95.8189) (size 0.6) (drill 0.3) (layers "F.Cu" "B.Cu") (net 3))
 (segment (start 118.4165 93.3102) (end 120.9252 95.8189) (width 0.2) (layer "B.Cu") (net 3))
 (segment (start 120.9252 95.8189) (end 126.0017 95.8189) (width 0.2) (layer "B.Cu") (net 3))
 (segment (start 93.66 94.4) (end 94.7498 93.3102) (width 0.2) (layer "B.Cu") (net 3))
 (segment (start 94.7498 93.3102) (end 118.4165 93.3102) (width 0.2) (layer "B.Cu") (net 3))
 (segment (start 109.735 109.64) (end 109.735 134.8174) (width 0.2) (layer "F.Cu") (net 8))
 (segment (start 109.735 109.64) (end 108.9 109.64) (width 0.2) (layer "F.Cu") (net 8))
 (segment (start 109.735 134.8174) (end 117.6338 142.7162) (width 0.2) (layer "F.Cu") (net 8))
 (segment (start 109.735 107.1) (end 108.9 107.1) (width 0.2) (layer "F.Cu") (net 12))
 (segment (start 98.5838 117.4162) (end 98.5838 123.6662) (width 0.2) (layer "B.Cu") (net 12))
 (segment (start 108.9 107.1) (end 98.5838 117.4162) (width 0.2) (layer "B.Cu") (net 12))
 (segment (start 109.735 104.56) (end 117.6338 112.4588) (width 0.2) (layer "F.Cu") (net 13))
 (segment (start 117.6338 112.4588) (end 117.6338 123.6662) (width 0.2) (layer "F.Cu") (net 13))
 (segment (start 108.9 104.56) (end 109.735 104.56) (width 0.2) (layer "F.Cu") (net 13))
 (segment (start 107.8173 103.1027) (end 107.8173 123.8804) (width 0.2) (layer "F.Cu") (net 14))
 (segment (start 107.8173 123.8804) (end 105.6504 126.0473) (width 0.2) (layer "F.Cu") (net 14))
 (segment (start 105.6504 126.0473) (end 105.6504 135.6496) (width 0.2) (layer "F.Cu") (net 14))
 (segment (start 109.735 102.02) (end 108.9 102.02) (width 0.2) (layer "F.Cu") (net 14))
 (segment (start 108.9 102.02) (end 107.8173 103.1027) (width 0.2) (layer "F.Cu") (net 14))
 (segment (start 105.6504 135.6496) (end 98.5838 142.7162) (width 0.2) (layer "F.Cu") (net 14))
 (segment (start 109.735 99.48) (end 108.9 99.48) (width 0.2) (layer "F.Cu") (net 15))
 (segment (start 93.66 104.56) (end 92.825 104.56) (width 0.2) (layer "F.Cu") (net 6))
 (segment (start 106.1831 103.29) (end 101.3057 108.1674) (width 0.2) (layer "B.Cu") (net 6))
 (segment (start 92.5937 107.5655) (end 92.5937 105.6263) (width 0.2) (layer "B.Cu") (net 6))
 (segment (start 114.8 101.6) (end 113.11 103.29) (width 0.2) (layer "B.Cu") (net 6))
 (segment (start 93.1956 108.1674) (end 92.5937 107.5655) (width 0.2) (layer "B.Cu") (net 6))
 (segment (start 113.11 103.29) (end 106.1831 103.29) (width 0.2) (layer "B.Cu") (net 6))
 (segment (start 92.5937 105.6263) (end 93.66 104.56) (width 0.2) (layer "B.Cu") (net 6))
 (segment (start 101.3057 108.1674) (end 93.1956 108.1674) (width 0.2) (layer "B.Cu") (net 6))
 (segment (start 93.66 109.64) (end 92.825 109.64) (width 0.2) (layer "F.Cu") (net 7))
 (segment (start 119.0004 101.6) (end 114.7704 105.83) (width 0.2) (layer "B.Cu") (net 7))
 (segment (start 104.0278 109.64) (end 93.66 109.64) (width 0.2) (layer "B.Cu") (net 7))
 (segment (start 129.3 101.6) (end 119.0004 101.6) (width 0.2) (layer "B.Cu") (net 7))
 (segment (start 114.7704 105.83) (end 107.8378 105.83) (width 0.2) (layer "B.Cu") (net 7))
 (segment (start 107.8378 105.83) (end 104.0278 109.64) (width 0.2) (layer "B.Cu") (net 7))
 (segment (start 93.66 107.1) (end 92.825 107.1) (width 0.2) (layer "F.Cu") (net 5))
 (segment (start 112.7616 95.8633) (end 113.4983 96.6) (width 0.2) (layer "B.Cu") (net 5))
 (segment (start 104.8967 95.8633) (end 112.7616 95.8633) (width 0.2) (layer "B.Cu") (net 5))
 (segment (start 93.66 107.1) (end 104.8967 95.8633) (width 0.2) (layer "B.Cu") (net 5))
 (segment (start 114.8 96.6) (end 113.4983 96.6) (width 0.2) (layer "B.Cu") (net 5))
 (segment (start 93.66 99.48) (end 92.825 99.48) (width 0.2) (layer "F.Cu") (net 10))
 (segment (start 93.66 96.94) (end 92.825 96.94) (width 0.2) (layer "F.Cu") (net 9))
 (segment (start 93.66 102.02) (end 92.825 102.02) (width 0.2) (layer "F.Cu") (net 11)))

